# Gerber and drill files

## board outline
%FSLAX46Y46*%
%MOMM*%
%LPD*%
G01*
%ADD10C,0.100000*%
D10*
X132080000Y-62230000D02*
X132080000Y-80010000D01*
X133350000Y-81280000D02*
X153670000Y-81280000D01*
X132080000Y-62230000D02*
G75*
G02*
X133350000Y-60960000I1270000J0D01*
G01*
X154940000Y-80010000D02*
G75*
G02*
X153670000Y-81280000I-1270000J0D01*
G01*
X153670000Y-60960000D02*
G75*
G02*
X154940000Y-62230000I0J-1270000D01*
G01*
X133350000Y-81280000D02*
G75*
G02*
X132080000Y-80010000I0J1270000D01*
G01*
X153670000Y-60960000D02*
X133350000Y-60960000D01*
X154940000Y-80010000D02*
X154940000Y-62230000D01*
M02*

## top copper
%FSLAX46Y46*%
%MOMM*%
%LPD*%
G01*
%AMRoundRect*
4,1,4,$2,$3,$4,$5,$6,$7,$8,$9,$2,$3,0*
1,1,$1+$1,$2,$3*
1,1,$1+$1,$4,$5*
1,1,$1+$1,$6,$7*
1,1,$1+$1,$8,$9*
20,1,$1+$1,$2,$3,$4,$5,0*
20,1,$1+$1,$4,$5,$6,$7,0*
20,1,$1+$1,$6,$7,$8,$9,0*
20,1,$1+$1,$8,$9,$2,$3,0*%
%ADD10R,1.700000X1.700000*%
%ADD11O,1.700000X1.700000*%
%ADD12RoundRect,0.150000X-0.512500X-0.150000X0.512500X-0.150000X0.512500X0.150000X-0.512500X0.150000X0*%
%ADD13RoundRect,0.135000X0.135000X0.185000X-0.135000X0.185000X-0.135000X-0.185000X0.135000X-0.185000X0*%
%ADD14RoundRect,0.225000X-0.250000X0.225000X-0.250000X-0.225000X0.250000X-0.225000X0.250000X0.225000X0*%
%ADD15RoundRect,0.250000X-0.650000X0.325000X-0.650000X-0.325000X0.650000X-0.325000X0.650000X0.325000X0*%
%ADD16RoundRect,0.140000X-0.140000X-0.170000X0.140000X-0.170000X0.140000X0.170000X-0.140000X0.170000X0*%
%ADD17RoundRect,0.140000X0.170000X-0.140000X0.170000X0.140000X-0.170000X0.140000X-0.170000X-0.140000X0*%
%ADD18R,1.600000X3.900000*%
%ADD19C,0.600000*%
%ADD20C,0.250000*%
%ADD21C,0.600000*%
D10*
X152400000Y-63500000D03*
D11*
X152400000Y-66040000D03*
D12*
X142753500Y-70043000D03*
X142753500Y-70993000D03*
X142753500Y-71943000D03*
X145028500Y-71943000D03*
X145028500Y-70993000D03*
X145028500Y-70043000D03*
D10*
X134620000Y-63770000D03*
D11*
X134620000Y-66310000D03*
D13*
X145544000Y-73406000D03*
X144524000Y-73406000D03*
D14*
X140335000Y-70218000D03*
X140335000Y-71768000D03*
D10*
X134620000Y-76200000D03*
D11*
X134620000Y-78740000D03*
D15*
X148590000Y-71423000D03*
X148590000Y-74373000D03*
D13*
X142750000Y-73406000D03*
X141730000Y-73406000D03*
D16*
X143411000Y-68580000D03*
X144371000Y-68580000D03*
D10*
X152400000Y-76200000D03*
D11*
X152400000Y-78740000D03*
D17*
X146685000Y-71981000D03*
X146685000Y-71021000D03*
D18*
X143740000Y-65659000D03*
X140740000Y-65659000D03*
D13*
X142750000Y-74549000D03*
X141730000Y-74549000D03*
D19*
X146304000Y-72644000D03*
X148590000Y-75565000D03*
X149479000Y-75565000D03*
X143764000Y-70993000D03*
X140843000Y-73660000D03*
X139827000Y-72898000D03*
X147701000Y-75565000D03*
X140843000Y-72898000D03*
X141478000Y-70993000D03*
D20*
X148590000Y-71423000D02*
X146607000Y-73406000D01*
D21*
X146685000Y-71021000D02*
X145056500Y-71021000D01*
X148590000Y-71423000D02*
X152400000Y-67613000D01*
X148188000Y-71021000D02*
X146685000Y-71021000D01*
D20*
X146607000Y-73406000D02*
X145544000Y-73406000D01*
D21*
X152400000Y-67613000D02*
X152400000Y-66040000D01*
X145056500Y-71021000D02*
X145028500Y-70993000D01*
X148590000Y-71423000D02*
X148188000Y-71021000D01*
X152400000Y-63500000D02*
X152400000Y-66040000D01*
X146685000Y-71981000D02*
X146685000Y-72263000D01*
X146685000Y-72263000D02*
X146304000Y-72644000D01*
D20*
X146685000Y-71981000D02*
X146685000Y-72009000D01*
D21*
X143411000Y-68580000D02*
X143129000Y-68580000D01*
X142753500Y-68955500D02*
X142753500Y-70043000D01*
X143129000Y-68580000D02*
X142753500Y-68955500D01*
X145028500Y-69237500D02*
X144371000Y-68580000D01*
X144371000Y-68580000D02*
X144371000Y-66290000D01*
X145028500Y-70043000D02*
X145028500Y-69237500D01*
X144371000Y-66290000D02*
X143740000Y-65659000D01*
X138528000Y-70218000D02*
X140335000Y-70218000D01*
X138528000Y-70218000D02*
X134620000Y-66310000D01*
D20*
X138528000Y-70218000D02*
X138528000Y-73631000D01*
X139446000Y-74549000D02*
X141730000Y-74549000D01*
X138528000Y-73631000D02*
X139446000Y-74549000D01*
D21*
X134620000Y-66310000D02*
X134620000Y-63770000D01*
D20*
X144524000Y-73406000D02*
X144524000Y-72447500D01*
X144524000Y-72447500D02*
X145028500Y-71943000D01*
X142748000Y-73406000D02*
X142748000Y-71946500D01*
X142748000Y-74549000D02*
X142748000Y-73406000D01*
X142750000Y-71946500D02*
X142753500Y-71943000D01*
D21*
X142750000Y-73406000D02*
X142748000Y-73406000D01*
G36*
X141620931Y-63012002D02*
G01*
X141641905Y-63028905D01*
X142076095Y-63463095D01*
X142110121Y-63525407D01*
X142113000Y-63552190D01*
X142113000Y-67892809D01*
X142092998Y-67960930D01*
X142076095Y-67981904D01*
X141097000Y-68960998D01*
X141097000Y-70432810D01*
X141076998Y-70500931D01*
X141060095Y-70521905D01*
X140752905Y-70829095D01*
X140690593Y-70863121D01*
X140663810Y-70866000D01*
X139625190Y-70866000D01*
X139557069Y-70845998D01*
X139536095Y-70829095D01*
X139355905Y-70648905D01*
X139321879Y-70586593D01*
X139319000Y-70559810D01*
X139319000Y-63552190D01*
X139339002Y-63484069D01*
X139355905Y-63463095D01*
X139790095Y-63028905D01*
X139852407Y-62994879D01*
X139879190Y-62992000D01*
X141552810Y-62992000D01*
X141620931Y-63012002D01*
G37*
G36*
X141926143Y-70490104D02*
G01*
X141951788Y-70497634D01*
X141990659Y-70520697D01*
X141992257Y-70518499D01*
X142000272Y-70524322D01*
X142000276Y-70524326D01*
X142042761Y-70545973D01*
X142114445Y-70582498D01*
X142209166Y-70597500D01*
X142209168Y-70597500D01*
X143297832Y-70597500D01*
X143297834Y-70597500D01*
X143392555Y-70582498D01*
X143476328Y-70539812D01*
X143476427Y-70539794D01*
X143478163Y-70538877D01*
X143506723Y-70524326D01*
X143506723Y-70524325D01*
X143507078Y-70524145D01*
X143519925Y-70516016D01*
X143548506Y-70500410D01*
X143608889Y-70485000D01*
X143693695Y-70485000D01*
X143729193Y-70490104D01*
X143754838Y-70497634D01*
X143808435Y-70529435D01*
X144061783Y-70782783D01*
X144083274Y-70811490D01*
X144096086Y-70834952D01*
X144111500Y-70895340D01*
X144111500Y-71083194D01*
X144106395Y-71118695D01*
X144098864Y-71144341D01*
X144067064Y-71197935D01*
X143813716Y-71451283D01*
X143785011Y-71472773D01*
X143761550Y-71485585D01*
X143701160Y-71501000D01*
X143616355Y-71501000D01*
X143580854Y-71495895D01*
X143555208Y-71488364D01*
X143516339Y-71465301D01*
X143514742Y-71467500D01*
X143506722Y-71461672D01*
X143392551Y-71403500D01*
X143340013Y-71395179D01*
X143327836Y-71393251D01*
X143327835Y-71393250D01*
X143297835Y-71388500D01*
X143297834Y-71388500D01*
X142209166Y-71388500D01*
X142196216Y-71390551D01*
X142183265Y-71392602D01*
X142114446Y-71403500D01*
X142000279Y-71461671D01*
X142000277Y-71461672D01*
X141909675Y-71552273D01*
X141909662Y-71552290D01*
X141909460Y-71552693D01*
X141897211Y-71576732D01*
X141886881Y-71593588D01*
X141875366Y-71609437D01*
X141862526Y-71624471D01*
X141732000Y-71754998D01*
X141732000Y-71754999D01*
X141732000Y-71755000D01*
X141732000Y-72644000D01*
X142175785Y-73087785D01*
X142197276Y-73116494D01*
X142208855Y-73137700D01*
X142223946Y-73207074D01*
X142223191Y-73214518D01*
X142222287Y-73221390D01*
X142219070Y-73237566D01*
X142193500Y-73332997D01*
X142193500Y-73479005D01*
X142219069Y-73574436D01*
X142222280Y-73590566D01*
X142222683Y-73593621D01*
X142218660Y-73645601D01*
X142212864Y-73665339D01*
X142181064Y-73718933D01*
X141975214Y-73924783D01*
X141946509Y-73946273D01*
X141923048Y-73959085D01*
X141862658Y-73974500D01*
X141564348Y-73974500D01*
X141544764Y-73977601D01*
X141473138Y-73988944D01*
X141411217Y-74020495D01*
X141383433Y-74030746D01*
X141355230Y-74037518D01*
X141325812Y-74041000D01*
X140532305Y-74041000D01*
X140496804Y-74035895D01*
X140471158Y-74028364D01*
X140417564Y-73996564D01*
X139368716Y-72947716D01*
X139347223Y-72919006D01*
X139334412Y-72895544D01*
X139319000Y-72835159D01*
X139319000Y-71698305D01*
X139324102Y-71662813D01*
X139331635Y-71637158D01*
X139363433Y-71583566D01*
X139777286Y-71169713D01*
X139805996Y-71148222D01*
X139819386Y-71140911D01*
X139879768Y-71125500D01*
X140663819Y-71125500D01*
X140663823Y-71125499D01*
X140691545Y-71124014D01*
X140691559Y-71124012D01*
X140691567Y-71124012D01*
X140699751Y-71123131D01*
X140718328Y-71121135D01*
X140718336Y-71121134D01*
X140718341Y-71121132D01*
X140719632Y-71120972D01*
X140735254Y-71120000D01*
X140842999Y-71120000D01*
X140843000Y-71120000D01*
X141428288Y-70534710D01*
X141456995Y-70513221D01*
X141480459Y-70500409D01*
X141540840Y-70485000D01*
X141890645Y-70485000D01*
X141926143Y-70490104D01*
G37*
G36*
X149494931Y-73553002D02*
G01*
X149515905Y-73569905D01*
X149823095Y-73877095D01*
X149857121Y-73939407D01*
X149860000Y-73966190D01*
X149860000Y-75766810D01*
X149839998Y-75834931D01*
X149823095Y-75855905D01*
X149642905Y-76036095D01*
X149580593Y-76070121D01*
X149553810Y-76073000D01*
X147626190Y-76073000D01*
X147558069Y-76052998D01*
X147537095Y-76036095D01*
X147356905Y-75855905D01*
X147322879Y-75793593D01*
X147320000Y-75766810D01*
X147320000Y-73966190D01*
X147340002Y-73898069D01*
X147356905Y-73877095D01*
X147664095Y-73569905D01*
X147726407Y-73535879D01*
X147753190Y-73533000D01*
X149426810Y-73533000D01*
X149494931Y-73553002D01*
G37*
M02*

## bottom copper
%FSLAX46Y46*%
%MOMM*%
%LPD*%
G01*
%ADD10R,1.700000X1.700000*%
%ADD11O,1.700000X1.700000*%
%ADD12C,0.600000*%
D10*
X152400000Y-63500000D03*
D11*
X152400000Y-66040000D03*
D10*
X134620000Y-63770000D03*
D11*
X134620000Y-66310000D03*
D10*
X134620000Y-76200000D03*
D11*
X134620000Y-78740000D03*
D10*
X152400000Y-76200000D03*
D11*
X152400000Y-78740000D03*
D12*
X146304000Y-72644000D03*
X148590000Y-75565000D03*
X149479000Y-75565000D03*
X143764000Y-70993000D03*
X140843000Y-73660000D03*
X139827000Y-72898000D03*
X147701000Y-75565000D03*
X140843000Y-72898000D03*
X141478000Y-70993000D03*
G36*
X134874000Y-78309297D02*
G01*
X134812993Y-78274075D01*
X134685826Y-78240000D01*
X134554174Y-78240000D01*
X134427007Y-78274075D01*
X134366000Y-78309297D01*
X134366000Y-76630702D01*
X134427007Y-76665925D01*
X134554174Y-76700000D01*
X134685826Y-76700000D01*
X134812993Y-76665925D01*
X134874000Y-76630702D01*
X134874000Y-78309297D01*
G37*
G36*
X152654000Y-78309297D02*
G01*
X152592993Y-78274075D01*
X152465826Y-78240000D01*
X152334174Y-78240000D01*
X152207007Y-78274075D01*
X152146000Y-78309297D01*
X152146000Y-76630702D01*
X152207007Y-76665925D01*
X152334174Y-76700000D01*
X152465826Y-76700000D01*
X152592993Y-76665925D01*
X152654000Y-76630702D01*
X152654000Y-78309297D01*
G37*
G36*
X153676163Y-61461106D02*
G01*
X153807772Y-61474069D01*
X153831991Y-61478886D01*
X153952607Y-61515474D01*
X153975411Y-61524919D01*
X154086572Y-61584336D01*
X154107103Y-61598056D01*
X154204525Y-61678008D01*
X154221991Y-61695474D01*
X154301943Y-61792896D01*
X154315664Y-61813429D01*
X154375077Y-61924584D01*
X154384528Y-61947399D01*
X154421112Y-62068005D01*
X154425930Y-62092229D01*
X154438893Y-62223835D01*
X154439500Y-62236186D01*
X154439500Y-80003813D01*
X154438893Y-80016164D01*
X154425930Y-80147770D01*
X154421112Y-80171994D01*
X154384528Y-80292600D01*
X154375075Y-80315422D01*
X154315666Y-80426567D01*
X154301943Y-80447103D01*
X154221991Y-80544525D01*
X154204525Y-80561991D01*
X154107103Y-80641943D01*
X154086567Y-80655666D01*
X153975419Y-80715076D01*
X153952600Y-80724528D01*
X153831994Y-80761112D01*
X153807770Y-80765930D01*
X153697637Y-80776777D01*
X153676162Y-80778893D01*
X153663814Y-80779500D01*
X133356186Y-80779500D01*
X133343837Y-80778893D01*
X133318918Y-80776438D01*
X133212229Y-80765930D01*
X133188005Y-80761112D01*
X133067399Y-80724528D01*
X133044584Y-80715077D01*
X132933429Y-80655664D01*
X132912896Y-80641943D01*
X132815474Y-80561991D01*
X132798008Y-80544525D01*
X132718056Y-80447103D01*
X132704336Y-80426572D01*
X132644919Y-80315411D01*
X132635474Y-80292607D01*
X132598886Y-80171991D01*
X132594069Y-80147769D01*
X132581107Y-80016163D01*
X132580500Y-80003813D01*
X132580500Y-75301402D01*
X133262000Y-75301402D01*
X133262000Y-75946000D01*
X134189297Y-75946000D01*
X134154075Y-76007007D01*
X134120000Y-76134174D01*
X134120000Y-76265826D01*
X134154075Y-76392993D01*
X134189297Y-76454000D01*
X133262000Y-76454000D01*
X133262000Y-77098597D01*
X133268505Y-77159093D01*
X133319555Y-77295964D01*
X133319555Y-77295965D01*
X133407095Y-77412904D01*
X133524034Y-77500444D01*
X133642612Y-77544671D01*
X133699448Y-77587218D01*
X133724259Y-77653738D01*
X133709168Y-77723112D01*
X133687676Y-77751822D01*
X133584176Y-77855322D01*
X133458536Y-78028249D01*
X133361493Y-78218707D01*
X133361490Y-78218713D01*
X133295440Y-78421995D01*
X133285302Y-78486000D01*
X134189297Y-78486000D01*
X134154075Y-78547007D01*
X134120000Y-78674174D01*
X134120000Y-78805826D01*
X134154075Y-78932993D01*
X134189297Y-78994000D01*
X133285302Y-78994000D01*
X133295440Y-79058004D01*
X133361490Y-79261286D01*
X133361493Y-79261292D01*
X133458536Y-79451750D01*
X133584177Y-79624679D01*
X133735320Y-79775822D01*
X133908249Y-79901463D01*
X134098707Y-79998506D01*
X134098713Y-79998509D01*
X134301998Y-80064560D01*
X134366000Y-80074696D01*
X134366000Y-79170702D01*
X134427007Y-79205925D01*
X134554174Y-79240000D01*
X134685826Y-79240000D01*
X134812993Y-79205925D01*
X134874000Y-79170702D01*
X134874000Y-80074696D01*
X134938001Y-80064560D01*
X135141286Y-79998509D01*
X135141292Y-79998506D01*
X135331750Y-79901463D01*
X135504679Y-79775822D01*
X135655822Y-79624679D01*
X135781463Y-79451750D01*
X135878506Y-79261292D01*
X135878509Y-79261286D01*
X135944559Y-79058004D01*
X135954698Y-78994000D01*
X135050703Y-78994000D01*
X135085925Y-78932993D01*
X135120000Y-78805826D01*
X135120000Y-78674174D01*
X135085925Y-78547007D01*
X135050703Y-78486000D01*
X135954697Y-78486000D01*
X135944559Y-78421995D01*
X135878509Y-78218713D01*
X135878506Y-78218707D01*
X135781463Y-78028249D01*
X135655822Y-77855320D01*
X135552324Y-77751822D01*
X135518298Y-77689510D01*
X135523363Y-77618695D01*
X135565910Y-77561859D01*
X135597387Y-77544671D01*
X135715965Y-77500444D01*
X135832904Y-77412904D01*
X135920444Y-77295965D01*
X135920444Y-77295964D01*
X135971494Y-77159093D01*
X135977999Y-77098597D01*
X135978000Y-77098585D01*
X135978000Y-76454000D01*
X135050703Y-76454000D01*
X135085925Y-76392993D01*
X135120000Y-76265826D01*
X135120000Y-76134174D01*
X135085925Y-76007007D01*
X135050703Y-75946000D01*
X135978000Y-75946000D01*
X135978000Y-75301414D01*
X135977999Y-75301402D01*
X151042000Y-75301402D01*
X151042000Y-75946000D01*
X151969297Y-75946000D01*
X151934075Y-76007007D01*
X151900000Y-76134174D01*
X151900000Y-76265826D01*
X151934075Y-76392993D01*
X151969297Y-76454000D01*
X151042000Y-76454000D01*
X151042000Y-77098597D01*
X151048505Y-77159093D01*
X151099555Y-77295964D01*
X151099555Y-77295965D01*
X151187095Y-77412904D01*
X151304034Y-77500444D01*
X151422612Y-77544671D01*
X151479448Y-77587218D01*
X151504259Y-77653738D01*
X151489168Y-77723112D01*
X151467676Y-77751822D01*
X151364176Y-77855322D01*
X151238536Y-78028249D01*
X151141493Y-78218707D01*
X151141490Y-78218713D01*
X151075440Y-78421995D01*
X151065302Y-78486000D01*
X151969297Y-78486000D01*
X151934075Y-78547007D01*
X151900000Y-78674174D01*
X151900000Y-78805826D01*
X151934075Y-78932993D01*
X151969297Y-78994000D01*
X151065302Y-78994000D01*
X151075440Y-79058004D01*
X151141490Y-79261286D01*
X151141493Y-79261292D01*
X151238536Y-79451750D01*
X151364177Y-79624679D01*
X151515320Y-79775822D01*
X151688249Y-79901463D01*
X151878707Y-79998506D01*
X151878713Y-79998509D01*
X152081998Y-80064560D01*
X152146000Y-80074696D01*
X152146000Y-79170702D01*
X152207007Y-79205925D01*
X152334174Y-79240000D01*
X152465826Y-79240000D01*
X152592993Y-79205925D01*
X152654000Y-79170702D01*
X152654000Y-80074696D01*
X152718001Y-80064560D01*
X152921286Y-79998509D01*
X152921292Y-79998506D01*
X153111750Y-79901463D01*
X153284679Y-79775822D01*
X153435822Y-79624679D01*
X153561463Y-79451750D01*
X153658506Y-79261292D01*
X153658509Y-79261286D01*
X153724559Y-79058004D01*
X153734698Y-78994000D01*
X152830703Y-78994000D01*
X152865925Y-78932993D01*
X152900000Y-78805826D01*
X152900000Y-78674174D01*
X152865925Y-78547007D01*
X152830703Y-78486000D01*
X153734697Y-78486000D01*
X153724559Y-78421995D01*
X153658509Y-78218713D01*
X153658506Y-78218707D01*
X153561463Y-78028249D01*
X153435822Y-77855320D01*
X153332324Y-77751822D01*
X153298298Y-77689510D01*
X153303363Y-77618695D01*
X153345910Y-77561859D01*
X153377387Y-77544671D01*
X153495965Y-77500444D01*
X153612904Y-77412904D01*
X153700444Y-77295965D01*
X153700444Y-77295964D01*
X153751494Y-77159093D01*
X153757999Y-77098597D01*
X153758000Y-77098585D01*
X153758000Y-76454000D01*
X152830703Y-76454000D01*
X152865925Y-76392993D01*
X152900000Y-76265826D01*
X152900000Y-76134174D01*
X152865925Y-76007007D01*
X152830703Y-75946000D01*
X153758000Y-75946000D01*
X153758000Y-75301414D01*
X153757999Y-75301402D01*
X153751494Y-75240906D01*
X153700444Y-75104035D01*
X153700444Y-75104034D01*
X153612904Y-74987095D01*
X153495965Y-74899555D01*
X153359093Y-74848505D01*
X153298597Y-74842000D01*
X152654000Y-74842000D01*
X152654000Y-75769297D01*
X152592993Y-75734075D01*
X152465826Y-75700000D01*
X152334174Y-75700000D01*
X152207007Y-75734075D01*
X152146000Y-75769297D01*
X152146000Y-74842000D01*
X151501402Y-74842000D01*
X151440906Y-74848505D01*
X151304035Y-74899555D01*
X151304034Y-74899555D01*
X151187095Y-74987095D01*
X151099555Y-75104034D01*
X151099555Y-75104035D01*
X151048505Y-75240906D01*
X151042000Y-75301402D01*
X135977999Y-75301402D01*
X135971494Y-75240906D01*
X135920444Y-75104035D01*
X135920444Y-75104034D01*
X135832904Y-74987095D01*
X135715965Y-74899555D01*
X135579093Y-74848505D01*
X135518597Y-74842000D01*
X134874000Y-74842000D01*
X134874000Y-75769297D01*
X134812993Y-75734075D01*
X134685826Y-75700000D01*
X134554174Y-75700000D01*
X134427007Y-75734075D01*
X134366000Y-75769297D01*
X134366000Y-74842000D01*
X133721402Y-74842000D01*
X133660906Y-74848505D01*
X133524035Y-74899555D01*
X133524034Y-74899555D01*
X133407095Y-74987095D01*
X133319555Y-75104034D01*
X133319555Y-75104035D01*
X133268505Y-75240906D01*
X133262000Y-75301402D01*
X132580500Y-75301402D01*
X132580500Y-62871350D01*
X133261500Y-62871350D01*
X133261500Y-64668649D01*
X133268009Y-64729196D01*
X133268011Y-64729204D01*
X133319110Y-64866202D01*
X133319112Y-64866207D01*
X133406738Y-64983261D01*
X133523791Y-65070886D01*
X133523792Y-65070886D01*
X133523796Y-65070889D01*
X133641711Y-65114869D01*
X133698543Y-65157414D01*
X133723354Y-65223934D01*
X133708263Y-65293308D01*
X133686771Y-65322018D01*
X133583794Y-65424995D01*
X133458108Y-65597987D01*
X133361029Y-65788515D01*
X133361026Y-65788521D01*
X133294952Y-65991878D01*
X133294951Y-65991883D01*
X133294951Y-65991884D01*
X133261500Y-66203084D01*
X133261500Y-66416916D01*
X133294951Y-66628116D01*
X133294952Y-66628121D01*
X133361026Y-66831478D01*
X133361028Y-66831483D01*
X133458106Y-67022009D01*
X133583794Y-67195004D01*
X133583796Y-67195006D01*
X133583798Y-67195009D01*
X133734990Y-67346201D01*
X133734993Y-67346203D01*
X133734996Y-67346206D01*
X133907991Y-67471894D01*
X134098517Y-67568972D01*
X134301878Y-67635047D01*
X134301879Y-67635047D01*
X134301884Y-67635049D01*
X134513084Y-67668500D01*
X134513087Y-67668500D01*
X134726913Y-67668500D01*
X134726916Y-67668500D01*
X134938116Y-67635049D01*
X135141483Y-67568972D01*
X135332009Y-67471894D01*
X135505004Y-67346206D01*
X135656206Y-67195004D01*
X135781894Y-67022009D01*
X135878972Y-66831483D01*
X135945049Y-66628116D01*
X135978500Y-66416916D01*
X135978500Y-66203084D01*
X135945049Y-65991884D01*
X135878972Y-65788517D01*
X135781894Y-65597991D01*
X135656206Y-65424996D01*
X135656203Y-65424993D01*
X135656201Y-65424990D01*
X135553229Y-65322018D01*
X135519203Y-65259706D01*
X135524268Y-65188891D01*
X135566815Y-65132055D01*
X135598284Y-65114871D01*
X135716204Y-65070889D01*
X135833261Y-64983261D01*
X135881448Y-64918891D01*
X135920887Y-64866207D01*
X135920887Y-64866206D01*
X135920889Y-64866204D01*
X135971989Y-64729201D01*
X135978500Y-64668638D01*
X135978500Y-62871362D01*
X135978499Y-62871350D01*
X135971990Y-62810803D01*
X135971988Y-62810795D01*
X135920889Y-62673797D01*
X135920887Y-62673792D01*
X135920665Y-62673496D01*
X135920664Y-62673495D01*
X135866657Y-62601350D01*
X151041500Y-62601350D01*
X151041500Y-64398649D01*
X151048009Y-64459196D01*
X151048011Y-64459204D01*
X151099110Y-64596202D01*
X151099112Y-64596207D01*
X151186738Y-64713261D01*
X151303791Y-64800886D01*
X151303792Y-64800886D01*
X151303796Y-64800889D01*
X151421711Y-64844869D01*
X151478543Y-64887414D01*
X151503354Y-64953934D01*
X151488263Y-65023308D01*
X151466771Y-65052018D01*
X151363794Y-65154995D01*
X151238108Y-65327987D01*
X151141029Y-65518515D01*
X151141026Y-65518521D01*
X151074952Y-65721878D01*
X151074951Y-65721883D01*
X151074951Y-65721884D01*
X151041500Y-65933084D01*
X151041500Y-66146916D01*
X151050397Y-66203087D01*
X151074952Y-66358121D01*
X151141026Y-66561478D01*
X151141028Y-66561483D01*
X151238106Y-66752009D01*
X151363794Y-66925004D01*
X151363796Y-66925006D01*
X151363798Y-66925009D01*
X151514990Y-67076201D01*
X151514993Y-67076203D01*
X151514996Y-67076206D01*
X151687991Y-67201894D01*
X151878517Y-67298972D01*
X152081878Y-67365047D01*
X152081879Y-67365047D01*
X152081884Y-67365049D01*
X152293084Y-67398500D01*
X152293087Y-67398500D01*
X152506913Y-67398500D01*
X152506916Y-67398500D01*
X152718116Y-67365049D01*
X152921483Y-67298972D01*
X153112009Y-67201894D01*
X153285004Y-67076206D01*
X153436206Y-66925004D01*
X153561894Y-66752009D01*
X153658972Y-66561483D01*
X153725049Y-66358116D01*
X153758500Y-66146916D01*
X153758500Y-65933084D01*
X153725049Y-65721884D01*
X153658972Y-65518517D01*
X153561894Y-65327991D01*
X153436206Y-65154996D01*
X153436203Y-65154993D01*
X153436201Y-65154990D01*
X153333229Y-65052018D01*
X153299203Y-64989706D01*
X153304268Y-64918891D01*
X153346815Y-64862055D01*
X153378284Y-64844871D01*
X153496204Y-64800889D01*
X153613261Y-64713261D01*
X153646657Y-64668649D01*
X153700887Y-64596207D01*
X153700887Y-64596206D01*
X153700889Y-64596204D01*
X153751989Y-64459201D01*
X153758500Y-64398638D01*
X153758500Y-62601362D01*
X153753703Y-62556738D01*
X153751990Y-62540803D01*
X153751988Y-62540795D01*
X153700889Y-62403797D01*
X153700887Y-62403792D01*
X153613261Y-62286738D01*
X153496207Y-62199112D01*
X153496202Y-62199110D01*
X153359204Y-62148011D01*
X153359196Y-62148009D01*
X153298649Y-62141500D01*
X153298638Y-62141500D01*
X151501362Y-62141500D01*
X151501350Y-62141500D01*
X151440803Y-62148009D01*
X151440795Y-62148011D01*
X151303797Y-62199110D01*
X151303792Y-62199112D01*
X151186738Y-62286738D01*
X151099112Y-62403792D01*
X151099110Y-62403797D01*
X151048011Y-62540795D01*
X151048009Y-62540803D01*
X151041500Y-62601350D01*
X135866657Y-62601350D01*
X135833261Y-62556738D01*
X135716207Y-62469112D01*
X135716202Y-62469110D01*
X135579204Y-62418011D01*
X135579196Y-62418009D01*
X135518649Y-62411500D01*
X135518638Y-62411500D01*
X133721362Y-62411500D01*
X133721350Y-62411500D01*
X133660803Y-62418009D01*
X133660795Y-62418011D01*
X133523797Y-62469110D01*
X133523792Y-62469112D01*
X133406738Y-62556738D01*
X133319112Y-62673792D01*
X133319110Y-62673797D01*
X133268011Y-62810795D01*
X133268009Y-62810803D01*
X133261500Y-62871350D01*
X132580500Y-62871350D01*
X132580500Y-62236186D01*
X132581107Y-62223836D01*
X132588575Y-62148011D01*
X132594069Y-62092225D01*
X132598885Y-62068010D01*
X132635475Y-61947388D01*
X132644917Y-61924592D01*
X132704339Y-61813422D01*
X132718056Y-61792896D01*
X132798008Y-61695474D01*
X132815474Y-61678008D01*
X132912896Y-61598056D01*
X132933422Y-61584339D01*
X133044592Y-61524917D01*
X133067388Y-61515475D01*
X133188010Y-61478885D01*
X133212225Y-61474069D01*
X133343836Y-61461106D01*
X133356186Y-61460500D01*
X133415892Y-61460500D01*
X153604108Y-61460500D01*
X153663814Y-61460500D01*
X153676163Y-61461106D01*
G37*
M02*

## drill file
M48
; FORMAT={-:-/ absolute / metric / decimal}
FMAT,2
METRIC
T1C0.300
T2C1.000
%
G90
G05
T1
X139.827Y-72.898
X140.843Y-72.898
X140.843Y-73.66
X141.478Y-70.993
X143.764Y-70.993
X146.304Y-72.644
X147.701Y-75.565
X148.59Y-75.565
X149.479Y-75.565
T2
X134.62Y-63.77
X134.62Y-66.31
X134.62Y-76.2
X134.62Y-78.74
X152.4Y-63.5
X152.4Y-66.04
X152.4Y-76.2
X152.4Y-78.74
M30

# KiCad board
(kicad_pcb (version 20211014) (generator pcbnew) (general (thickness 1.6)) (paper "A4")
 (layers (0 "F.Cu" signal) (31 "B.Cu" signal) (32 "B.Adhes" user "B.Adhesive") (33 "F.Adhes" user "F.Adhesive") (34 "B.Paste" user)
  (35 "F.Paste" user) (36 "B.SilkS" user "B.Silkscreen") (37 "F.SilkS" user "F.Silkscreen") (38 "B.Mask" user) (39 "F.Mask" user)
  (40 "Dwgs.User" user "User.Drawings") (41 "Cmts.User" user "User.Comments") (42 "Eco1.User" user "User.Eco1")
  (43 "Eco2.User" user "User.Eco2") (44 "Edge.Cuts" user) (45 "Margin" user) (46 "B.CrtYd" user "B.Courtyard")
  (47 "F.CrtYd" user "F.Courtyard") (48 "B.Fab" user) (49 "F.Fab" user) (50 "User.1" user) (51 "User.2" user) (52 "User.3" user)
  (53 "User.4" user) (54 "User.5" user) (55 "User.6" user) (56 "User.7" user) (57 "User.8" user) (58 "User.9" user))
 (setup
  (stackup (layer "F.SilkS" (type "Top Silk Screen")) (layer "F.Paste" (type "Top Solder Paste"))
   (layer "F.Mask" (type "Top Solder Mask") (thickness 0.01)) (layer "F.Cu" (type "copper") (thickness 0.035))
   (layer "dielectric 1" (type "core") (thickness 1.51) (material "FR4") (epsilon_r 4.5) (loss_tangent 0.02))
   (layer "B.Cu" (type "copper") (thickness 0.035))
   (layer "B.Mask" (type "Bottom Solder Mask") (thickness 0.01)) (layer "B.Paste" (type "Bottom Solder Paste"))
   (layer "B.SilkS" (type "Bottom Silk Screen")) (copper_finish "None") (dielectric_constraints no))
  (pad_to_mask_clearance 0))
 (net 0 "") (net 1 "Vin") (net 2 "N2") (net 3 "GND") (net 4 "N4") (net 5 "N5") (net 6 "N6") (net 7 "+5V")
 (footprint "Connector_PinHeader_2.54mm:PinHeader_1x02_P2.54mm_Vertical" (layer "F.Cu") (at 152.4 63.5)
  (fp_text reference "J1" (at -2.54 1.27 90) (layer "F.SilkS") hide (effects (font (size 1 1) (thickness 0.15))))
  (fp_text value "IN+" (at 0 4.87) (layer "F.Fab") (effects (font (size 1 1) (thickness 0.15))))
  (pad "1" thru_hole rect (at 0 0) (size 1.7 1.7) (drill 1) (layers *.Cu *.Mask) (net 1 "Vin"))
  (pad "2" thru_hole oval (at 0 2.54) (size 1.7 1.7) (drill 1) (layers *.Cu *.Mask) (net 1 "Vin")))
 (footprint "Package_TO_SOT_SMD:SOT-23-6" (layer "F.Cu") (at 143.891 70.993)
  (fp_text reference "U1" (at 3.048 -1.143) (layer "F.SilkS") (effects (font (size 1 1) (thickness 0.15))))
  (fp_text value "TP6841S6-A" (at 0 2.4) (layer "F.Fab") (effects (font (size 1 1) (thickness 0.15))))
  (pad "1" smd roundrect (at -1.1375 -0.95) (size 1.325 0.6) (layers "F.Cu" "F.Paste" "F.Mask") (roundrect_rratio 0.25) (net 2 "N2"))
  (pad "2" smd roundrect (at -1.1375 0) (size 1.325 0.6) (layers "F.Cu" "F.Paste" "F.Mask") (roundrect_rratio 0.25) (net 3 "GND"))
  (pad "3" smd roundrect (at -1.1375 0.95) (size 1.325 0.6) (layers "F.Cu" "F.Paste" "F.Mask") (roundrect_rratio 0.25) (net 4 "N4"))
  (pad "4" smd roundrect (at 1.1375 0.95) (size 1.325 0.6) (layers "F.Cu" "F.Paste" "F.Mask") (roundrect_rratio 0.25) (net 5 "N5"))
  (pad "5" smd roundrect (at 1.1375 0) (size 1.325 0.6) (layers "F.Cu" "F.Paste" "F.Mask") (roundrect_rratio 0.25) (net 1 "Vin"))
  (pad "6" smd roundrect (at 1.1375 -0.95) (size 1.325 0.6) (layers "F.Cu" "F.Paste" "F.Mask") (roundrect_rratio 0.25) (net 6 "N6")))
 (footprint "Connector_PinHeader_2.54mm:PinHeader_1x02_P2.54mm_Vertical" (layer "F.Cu") (at 134.62 63.77)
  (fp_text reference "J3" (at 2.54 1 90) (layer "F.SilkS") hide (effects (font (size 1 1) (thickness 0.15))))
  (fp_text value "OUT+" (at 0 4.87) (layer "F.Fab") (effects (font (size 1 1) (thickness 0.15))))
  (pad "1" thru_hole rect (at 0 0) (size 1.7 1.7) (drill 1) (layers *.Cu *.Mask) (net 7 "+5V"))
  (pad "2" thru_hole oval (at 0 2.54) (size 1.7 1.7) (drill 1) (layers *.Cu *.Mask) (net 7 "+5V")))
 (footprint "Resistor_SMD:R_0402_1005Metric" (layer "F.Cu") (at 145.034 73.406 180)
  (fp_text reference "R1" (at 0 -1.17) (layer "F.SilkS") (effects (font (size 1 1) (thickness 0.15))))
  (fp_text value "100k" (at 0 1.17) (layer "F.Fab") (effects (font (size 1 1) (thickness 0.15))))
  (pad "1" smd roundrect (at -0.51 0 180) (size 0.54 0.64) (layers "F.Cu" "F.Paste" "F.Mask") (roundrect_rratio 0.25) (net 1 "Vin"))
  (pad "2" smd roundrect (at 0.51 0 180) (size 0.54 0.64) (layers "F.Cu" "F.Paste" "F.Mask") (roundrect_rratio 0.25) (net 5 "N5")))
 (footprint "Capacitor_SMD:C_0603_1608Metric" (layer "F.Cu") (at 140.335 70.993 -90)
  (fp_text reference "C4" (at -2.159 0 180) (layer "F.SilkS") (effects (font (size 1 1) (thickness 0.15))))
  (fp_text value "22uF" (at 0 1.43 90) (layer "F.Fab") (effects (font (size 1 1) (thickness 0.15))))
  (pad "1" smd roundrect (at -0.775 0 270) (size 0.9 0.95) (layers "F.Cu" "F.Paste" "F.Mask") (roundrect_rratio 0.25) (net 7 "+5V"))
  (pad "2" smd roundrect (at 0.775 0 270) (size 0.9 0.95) (layers "F.Cu" "F.Paste" "F.Mask") (roundrect_rratio 0.25) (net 3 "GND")))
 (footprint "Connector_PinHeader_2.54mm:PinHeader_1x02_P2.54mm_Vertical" (layer "F.Cu") (at 134.62 76.2)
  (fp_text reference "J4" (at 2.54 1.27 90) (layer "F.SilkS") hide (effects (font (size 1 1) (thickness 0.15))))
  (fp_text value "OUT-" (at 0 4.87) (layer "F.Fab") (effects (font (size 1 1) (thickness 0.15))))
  (pad "1" thru_hole rect (at 0 0) (size 1.7 1.7) (drill 1) (layers *.Cu *.Mask) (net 3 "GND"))
  (pad "2" thru_hole oval (at 0 2.54) (size 1.7 1.7) (drill 1) (layers *.Cu *.Mask) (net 3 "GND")))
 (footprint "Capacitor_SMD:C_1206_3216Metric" (layer "F.Cu") (at 148.59 72.898 -90)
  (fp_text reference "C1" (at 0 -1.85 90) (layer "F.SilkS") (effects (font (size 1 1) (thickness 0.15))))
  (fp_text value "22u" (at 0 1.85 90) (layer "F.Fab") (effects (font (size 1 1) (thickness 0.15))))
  (pad "1" smd roundrect (at -1.475 0 270) (size 1.15 1.8) (layers "F.Cu" "F.Paste" "F.Mask") (roundrect_rratio 0.217391) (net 1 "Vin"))
  (pad "2" smd roundrect (at 1.475 0 270) (size 1.15 1.8) (layers "F.Cu" "F.Paste" "F.Mask") (roundrect_rratio 0.217391) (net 3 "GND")))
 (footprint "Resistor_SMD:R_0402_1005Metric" (layer "F.Cu") (at 142.24 73.406 180)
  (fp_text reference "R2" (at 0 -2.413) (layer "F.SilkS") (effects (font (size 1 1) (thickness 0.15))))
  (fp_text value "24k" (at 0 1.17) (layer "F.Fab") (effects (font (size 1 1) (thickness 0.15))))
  (pad "1" smd roundrect (at -0.51 0 180) (size 0.54 0.64) (layers "F.Cu" "F.Paste" "F.Mask") (roundrect_rratio 0.25) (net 4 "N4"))
  (pad "2" smd roundrect (at 0.51 0 180) (size 0.54 0.64) (layers "F.Cu" "F.Paste" "F.Mask") (roundrect_rratio 0.25) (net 3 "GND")))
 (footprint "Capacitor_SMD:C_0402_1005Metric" (layer "F.Cu") (at 143.891 68.58)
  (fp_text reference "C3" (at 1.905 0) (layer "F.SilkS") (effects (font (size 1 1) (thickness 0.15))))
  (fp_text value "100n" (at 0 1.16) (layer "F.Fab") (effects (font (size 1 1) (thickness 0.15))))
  (pad "1" smd roundrect (at -0.48 0) (size 0.56 0.62) (layers "F.Cu" "F.Paste" "F.Mask") (roundrect_rratio 0.25) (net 2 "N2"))
  (pad "2" smd roundrect (at 0.48 0) (size 0.56 0.62) (layers "F.Cu" "F.Paste" "F.Mask") (roundrect_rratio 0.25) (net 6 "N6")))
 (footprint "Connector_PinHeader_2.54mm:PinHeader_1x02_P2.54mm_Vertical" (layer "F.Cu") (at 152.4 76.2)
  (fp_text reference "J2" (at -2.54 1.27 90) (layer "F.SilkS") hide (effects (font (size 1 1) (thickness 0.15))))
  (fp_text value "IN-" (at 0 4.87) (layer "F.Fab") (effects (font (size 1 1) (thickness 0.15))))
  (pad "1" thru_hole rect (at 0 0) (size 1.7 1.7) (drill 1) (layers *.Cu *.Mask) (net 3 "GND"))
  (pad "2" thru_hole oval (at 0 2.54) (size 1.7 1.7) (drill 1) (layers *.Cu *.Mask) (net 3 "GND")))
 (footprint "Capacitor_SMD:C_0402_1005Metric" (layer "F.Cu") (at 146.685 71.501 90)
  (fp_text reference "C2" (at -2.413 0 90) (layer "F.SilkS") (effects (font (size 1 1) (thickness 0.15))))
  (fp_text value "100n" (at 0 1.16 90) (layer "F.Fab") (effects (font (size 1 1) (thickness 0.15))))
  (pad "1" smd roundrect (at -0.48 0 90) (size 0.56 0.62) (layers "F.Cu" "F.Paste" "F.Mask") (roundrect_rratio 0.25) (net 3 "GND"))
  (pad "2" smd roundrect (at 0.48 0 90) (size 0.56 0.62) (layers "F.Cu" "F.Paste" "F.Mask") (roundrect_rratio 0.25) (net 1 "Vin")))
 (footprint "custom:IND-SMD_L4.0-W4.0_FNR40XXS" (layer "F.Cu") (at 142.24 65.659 180)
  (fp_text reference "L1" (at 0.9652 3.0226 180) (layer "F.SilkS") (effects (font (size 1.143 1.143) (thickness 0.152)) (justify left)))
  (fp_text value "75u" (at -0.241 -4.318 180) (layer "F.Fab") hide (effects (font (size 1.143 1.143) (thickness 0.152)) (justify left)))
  (pad "1" smd rect (at -1.5 0 180) (size 1.6 3.9) (layers "F.Cu" "F.Paste" "F.Mask") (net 6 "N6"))
  (pad "2" smd rect (at 1.5 0 180) (size 1.6 3.9) (layers "F.Cu" "F.Paste" "F.Mask") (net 7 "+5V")))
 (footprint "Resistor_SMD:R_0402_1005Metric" (layer "F.Cu") (at 142.24 74.549 180)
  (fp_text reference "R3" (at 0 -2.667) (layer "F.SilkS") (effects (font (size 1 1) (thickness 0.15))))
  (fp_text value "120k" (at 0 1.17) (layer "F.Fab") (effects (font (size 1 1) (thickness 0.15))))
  (pad "1" smd roundrect (at -0.51 0 180) (size 0.54 0.64) (layers "F.Cu" "F.Paste" "F.Mask") (roundrect_rratio 0.25) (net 4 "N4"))
  (pad "2" smd roundrect (at 0.51 0 180) (size 0.54 0.64) (layers "F.Cu" "F.Paste" "F.Mask") (roundrect_rratio 0.25) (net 7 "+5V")))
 (gr_line (start 132.08 62.23) (end 132.08 80.01) (layer "Edge.Cuts") (width 0.1))
 (gr_line (start 133.35 81.28) (end 153.67 81.28) (layer "Edge.Cuts") (width 0.1))
 (gr_arc (start 132.08 62.23) (mid 132.451974 61.331974) (end 133.35 60.96) (layer "Edge.Cuts") (width 0.1))
 (gr_arc (start 154.94 80.01) (mid 154.568026 80.908026) (end 153.67 81.28) (layer "Edge.Cuts") (width 0.1))
 (gr_arc (start 153.67 60.96) (mid 154.568026 61.331974) (end 154.94 62.23) (layer "Edge.Cuts") (width 0.1))
 (gr_arc (start 133.35 81.28) (mid 132.451974 80.908026) (end 132.08 80.01) (layer "Edge.Cuts") (width 0.1))
 (gr_line (start 153.67 60.96) (end 133.35 60.96) (layer "Edge.Cuts") (width 0.1))
 (gr_line (start 154.94 80.01) (end 154.94 62.23) (layer "Edge.Cuts") (width 0.1))
 (segment (start 148.59 71.423) (end 146.607 73.406) (width 0.25) (layer "F.Cu") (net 1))
 (segment (start 146.685 71.021) (end 145.0565 71.021) (width 0.6) (layer "F.Cu") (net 1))
 (segment (start 148.59 71.423) (end 152.4 67.613) (width 0.6) (layer "F.Cu") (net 1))
 (segment (start 148.188 71.021) (end 146.685 71.021) (width 0.6) (layer "F.Cu") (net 1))
 (segment (start 146.607 73.406) (end 145.544 73.406) (width 0.25) (layer "F.Cu") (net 1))
 (segment (start 152.4 67.613) (end 152.4 66.04) (width 0.6) (layer "F.Cu") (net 1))
 (segment (start 145.0565 71.021) (end 145.0285 70.993) (width 0.6) (layer "F.Cu") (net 1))
 (segment (start 148.59 71.423) (end 148.188 71.021) (width 0.6) (layer "F.Cu") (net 1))
 (segment (start 152.4 63.5) (end 152.4 66.04) (width 0.6) (layer "F.Cu") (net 1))
 (segment (start 146.685 71.981) (end 146.685 72.263) (width 0.6) (layer "F.Cu") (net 3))
 (segment (start 146.685 72.263) (end 146.304 72.644) (width 0.6) (layer "F.Cu") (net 3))
 (segment (start 146.685 71.981) (end 146.685 72.009) (width 0.25) (layer "F.Cu") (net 3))
 (via (at 146.304 72.644) (size 0.6) (drill 0.3) (layers "F.Cu" "B.Cu") (free) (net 3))
 (via (at 148.59 75.565) (size 0.6) (drill 0.3) (layers "F.Cu" "B.Cu") (free) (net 3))
 (via (at 149.479 75.565) (size 0.6) (drill 0.3) (layers "F.Cu" "B.Cu") (free) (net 3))
 (via (at 143.764 70.993) (size 0.6) (drill 0.3) (layers "F.Cu" "B.Cu") (free) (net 3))
 (via (at 140.843 73.66) (size 0.6) (drill 0.3) (layers "F.Cu" "B.Cu") (free) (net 3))
 (via (at 139.827 72.898) (size 0.6) (drill 0.3) (layers "F.Cu" "B.Cu") (free) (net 3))
 (via (at 147.701 75.565) (size 0.6) (drill 0.3) (layers "F.Cu" "B.Cu") (free) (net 3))
 (via (at 140.843 72.898) (size 0.6) (drill 0.3) (layers "F.Cu" "B.Cu") (free) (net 3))
 (via (at 141.478 70.993) (size 0.6) (drill 0.3) (layers "F.Cu" "B.Cu") (free) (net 3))
 (segment (start 143.411 68.58) (end 143.129 68.58) (width 0.6) (layer "F.Cu") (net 2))
 (segment (start 142.7535 68.9555) (end 142.7535 70.043) (width 0.6) (layer "F.Cu") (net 2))
 (segment (start 143.129 68.58) (end 142.7535 68.9555) (width 0.6) (layer "F.Cu") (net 2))
 (segment (start 145.0285 69.2375) (end 144.371 68.58) (width 0.6) (layer "F.Cu") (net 6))
 (segment (start 144.371 68.58) (end 144.371 66.29) (width 0.6) (layer "F.Cu") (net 6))
 (segment (start 145.0285 70.043) (end 145.0285 69.2375) (width 0.6) (layer "F.Cu") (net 6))
 (segment (start 144.371 66.29) (end 143.74 65.659) (width 0.6) (layer "F.Cu") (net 6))
 (segment (start 138.528 70.218) (end 140.335 70.218) (width 0.6) (layer "F.Cu") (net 7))
 (segment (start 138.528 70.218) (end 134.62 66.31) (width 0.6) (layer "F.Cu") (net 7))
 (segment (start 138.528 70.218) (end 138.528 73.631) (width 0.25) (layer "F.Cu") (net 7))
 (segment (start 139.446 74.549) (end 141.73 74.549) (width 0.25) (layer "F.Cu") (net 7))
 (segment (start 138.528 73.631) (end 139.446 74.549) (width 0.25) (layer "F.Cu") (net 7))
 (segment (start 134.62 66.31) (end 134.62 63.77) (width 0.6) (layer "F.Cu") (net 7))
 (segment (start 144.524 73.406) (end 144.524 72.4475) (width 0.25) (layer "F.Cu") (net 5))
 (segment (start 144.524 72.4475) (end 145.0285 71.943) (width 0.25) (layer "F.Cu") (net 5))
 (segment (start 142.748 73.406) (end 142.748 71.9465) (width 0.25) (layer "F.Cu") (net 4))
 (segment (start 142.748 74.549) (end 142.748 73.406) (width 0.25) (layer "F.Cu") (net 4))
 (segment (start 142.75 71.9465) (end 142.7535 71.943) (width 0.25) (layer "F.Cu") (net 4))
 (segment (start 142.75 73.406) (end 142.748 73.406) (width 0.6) (layer "F.Cu") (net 4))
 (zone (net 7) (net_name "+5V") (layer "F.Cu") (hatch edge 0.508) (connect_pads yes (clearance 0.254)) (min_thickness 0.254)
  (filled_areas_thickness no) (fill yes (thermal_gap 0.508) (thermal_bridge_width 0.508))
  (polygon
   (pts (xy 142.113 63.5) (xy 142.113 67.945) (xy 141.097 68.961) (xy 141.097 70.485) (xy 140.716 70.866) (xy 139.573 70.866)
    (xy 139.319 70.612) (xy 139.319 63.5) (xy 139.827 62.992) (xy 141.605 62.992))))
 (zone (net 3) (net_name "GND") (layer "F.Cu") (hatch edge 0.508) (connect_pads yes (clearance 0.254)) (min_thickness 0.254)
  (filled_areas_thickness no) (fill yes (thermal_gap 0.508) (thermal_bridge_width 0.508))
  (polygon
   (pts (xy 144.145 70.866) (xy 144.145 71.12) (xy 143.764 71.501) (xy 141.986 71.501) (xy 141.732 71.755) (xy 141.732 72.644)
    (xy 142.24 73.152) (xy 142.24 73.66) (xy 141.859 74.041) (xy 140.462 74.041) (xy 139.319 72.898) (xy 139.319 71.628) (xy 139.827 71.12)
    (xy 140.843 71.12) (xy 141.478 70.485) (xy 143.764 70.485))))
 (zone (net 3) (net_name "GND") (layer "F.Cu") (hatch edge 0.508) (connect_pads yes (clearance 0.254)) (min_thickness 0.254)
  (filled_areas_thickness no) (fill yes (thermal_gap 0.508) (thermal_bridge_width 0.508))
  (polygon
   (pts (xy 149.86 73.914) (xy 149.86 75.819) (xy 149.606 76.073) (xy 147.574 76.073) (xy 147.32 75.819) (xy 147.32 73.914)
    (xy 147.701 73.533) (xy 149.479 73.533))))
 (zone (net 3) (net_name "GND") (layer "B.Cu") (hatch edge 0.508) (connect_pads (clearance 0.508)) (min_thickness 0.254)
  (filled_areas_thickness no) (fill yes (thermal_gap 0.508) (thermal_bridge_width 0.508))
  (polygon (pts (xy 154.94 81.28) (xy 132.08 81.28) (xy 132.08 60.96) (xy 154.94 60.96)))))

